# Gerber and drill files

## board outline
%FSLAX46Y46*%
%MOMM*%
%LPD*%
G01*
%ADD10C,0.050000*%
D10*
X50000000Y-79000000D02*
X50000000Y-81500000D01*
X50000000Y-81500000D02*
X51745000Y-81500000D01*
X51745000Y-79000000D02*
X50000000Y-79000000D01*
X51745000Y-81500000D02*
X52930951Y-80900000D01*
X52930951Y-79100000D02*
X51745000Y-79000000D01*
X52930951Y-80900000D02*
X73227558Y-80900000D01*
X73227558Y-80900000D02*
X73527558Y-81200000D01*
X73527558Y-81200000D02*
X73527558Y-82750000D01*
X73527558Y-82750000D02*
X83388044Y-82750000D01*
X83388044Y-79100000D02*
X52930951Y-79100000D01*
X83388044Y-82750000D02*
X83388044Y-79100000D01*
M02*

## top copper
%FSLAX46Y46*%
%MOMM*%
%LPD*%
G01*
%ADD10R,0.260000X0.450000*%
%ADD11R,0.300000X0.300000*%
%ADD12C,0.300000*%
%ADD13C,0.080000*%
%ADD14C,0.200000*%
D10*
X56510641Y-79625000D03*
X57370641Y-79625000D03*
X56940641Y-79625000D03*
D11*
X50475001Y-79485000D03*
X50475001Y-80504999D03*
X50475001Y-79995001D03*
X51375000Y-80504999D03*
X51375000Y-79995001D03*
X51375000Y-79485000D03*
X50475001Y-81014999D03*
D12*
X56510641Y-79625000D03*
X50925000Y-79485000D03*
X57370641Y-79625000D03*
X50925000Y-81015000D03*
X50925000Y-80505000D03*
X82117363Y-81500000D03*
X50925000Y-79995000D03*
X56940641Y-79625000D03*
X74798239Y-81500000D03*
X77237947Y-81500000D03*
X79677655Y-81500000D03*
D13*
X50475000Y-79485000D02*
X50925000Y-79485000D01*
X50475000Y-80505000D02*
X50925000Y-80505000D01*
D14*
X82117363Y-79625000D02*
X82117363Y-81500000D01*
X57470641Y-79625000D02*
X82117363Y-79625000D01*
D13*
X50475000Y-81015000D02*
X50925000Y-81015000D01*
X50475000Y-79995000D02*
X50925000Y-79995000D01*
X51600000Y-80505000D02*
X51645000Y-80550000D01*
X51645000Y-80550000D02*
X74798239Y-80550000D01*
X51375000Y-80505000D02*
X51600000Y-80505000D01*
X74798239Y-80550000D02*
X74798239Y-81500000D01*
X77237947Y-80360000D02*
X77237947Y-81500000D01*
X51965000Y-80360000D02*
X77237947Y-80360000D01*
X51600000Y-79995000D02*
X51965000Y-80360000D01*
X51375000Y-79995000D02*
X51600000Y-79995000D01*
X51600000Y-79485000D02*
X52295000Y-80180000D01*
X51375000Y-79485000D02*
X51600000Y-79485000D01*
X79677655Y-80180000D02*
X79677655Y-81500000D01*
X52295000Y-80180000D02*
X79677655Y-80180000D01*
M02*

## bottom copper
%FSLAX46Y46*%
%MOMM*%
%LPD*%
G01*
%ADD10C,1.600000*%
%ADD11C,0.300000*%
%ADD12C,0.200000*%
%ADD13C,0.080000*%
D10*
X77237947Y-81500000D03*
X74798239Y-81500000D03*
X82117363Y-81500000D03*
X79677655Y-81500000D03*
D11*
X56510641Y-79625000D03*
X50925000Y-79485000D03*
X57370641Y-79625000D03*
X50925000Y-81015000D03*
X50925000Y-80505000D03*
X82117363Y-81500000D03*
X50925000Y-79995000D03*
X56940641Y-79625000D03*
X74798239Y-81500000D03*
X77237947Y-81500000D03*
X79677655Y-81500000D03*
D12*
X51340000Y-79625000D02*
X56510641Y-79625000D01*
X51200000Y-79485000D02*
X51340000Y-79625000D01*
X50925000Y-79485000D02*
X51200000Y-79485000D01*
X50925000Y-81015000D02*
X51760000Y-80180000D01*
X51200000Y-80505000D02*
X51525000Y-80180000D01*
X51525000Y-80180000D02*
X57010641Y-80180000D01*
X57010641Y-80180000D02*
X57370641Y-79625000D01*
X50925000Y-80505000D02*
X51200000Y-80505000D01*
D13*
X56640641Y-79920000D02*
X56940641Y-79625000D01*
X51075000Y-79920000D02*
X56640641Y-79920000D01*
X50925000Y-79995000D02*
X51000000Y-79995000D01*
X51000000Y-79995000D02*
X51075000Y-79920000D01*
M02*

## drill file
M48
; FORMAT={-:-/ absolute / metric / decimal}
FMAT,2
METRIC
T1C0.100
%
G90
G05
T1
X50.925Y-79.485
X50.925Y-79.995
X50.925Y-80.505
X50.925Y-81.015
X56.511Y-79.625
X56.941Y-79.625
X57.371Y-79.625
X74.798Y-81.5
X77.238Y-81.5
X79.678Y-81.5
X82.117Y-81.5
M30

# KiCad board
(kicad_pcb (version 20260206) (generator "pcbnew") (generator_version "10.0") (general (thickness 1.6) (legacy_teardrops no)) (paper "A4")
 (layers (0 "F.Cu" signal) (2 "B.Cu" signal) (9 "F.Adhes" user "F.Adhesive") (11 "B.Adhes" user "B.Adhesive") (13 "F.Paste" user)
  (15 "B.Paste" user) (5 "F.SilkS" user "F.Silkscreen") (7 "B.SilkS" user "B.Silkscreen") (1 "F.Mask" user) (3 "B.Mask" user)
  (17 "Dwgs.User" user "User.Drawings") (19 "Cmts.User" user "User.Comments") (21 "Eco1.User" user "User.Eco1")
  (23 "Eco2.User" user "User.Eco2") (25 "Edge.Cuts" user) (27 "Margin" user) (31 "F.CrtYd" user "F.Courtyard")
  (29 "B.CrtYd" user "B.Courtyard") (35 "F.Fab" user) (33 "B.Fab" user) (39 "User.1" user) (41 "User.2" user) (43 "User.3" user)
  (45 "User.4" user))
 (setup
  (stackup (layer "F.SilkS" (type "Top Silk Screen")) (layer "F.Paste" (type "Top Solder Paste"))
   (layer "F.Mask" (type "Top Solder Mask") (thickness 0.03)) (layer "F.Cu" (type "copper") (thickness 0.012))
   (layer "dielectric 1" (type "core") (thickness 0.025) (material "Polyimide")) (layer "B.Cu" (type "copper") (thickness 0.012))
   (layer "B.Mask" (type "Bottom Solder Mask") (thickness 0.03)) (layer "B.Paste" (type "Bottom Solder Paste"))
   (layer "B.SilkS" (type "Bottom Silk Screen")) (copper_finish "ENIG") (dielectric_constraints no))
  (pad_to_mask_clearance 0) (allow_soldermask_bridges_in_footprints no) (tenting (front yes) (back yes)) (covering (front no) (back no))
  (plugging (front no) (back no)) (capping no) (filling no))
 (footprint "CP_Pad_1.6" (layer "F.Cu") (at 74.798239 81.5)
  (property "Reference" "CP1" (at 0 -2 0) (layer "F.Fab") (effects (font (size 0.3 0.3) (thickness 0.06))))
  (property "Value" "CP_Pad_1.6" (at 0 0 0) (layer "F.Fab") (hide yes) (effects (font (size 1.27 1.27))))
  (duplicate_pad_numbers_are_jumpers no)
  (pad "1" smd circle (at 0 0) (size 1.6 1.6) (layers "B.Cu" "B.Mask") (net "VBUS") (solder_mask_margin 0.1)))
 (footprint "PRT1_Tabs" (layer "F.Cu") (at 56.940641 79.625)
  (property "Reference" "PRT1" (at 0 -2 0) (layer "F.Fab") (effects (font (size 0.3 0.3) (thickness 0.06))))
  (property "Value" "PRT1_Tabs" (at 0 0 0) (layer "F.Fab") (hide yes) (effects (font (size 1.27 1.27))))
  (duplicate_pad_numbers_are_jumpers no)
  (pad "1" smd rect (at -0.43 0) (size 0.26 0.45) (layers "F.Cu" "F.Mask") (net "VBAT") (solder_mask_margin 0.05) (thermal_bridge_angle 45))
  (pad "2" smd rect (at 0.43 0) (size 0.26 0.45) (layers "F.Cu" "F.Mask") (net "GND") (solder_mask_margin 0.05) (thermal_bridge_angle 45))
  (pad "3" smd rect (at 0 0) (size 0.26 0.45) (layers "F.Cu" "F.Mask") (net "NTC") (solder_mask_margin 0.05) (thermal_bridge_angle 45)))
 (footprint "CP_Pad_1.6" (layer "F.Cu") (at 77.237947 81.5)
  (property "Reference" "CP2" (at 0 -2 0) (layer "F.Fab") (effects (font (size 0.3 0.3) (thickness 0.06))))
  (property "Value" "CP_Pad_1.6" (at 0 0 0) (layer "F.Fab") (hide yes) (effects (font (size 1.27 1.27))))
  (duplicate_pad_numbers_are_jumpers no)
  (pad "1" smd circle (at 0 0) (size 1.6 1.6) (layers "B.Cu" "B.Mask") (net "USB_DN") (solder_mask_margin 0.1)))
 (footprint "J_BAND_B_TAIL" (layer "F.Cu") (at 50.9 80.25)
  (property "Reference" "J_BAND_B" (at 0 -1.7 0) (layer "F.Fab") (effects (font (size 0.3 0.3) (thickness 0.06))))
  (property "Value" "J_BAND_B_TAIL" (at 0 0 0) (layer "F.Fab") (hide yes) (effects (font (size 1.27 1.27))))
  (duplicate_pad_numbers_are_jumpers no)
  (pad "1" smd rect (at -0.424999 -0.765) (size 0.3 0.3) (layers "F.Cu" "F.Mask") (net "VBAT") (solder_mask_margin 0.05)
   (thermal_bridge_angle 45))
  (pad "2" smd rect (at -0.424999 0.254999) (size 0.3 0.3) (layers "F.Cu" "F.Mask") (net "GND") (solder_mask_margin 0.05)
   (thermal_bridge_angle 45))
  (pad "3" smd rect (at -0.424999 -0.254999) (size 0.3 0.3) (layers "F.Cu" "F.Mask") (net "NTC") (solder_mask_margin 0.05)
   (thermal_bridge_angle 45))
  (pad "4" smd rect (at 0.475 0.254999) (size 0.3 0.3) (layers "F.Cu" "F.Mask") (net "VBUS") (solder_mask_margin 0.05)
   (thermal_bridge_angle 45))
  (pad "5" smd rect (at 0.475 -0.254999) (size 0.3 0.3) (layers "F.Cu" "F.Mask") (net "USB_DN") (solder_mask_margin 0.05)
   (thermal_bridge_angle 45))
  (pad "6" smd rect (at 0.475 -0.765) (size 0.3 0.3) (layers "F.Cu" "F.Mask") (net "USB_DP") (solder_mask_margin 0.05)
   (thermal_bridge_angle 45))
  (pad "7" smd rect (at -0.424999 0.764999) (size 0.3 0.3) (layers "F.Cu" "F.Mask") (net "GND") (solder_mask_margin 0.05)
   (thermal_bridge_angle 45)))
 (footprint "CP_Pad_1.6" (layer "F.Cu") (at 82.117363 81.5)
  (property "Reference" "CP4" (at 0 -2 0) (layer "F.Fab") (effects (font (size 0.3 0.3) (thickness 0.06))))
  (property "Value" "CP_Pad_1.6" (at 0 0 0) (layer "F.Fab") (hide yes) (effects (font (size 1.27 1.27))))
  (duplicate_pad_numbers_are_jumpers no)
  (pad "1" smd circle (at 0 0) (size 1.6 1.6) (layers "B.Cu" "B.Mask") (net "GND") (solder_mask_margin 0.1)))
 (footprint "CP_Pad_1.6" (layer "F.Cu") (at 79.677655 81.5)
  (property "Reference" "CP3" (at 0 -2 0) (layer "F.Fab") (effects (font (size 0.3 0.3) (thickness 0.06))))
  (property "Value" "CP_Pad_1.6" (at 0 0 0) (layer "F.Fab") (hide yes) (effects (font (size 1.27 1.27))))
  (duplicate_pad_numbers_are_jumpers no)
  (pad "1" smd circle (at 0 0) (size 1.6 1.6) (layers "B.Cu" "B.Mask") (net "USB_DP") (solder_mask_margin 0.1)))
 (gr_line (start 50 79) (end 50 81.5) (stroke (width 0.05) (type default)) (layer "Edge.Cuts"))
 (gr_line (start 50 81.5) (end 51.745 81.5) (stroke (width 0.05) (type default)) (layer "Edge.Cuts"))
 (gr_line (start 51.745 79) (end 50 79) (stroke (width 0.05) (type default)) (layer "Edge.Cuts"))
 (gr_line (start 51.745 81.5) (end 52.930951 80.9) (stroke (width 0.05) (type default)) (layer "Edge.Cuts"))
 (gr_line (start 52.930951 79.1) (end 51.745 79) (stroke (width 0.05) (type default)) (layer "Edge.Cuts"))
 (gr_line (start 52.930951 80.9) (end 73.227558 80.9) (stroke (width 0.05) (type default)) (layer "Edge.Cuts"))
 (gr_line (start 73.227558 80.9) (end 73.527558 81.2) (stroke (width 0.05) (type default)) (layer "Edge.Cuts"))
 (gr_line (start 73.527558 81.2) (end 73.527558 82.75) (stroke (width 0.05) (type default)) (layer "Edge.Cuts"))
 (gr_line (start 73.527558 82.75) (end 83.388044 82.75) (stroke (width 0.05) (type default)) (layer "Edge.Cuts"))
 (gr_line (start 83.388044 79.1) (end 52.930951 79.1) (stroke (width 0.05) (type default)) (layer "Edge.Cuts"))
 (gr_line (start 83.388044 82.75) (end 83.388044 79.1) (stroke (width 0.05) (type default)) (layer "Edge.Cuts"))
 (segment (start 50.475 79.485) (end 50.925 79.485) (width 0.08) (layer "F.Cu") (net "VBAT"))
 (via (at 56.510641 79.625) (size 0.3) (drill 0.1) (layers "F.Cu" "B.Cu") (tenting (front yes) (back yes)) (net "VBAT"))
 (via (at 50.925 79.485) (size 0.3) (drill 0.1) (layers "F.Cu" "B.Cu") (tenting (front yes) (back yes)) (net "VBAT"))
 (segment (start 51.2 79.485) (end 51.34 79.625) (width 0.2) (layer "B.Cu") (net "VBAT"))
 (segment (start 51.34 79.625) (end 56.510641 79.625) (width 0.2) (layer "B.Cu") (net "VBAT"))
 (segment (start 50.925 79.485) (end 51.2 79.485) (width 0.2) (layer "B.Cu") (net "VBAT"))
 (segment (start 82.117363 79.625) (end 82.117363 81.5) (width 0.2) (layer "F.Cu") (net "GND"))
 (segment (start 50.475 80.505) (end 50.925 80.505) (width 0.08) (layer "F.Cu") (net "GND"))
 (segment (start 57.470641 79.625) (end 82.117363 79.625) (width 0.2) (layer "F.Cu") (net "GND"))
 (segment (start 50.475 81.015) (end 50.925 81.015) (width 0.08) (layer "F.Cu") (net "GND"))
 (via (at 50.925 81.015) (size 0.3) (drill 0.1) (layers "F.Cu" "B.Cu") (tenting (front yes) (back yes)) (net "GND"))
 (via (at 57.370641 79.625) (size 0.3) (drill 0.1) (layers "F.Cu" "B.Cu") (tenting (front yes) (back yes)) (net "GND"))
 (via (at 82.117363 81.5) (size 0.3) (drill 0.1) (layers "F.Cu" "B.Cu") (tenting (front yes) (back yes)) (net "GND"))
 (via (at 50.925 80.505) (size 0.3) (drill 0.1) (layers "F.Cu" "B.Cu") (tenting (front yes) (back yes)) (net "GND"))
 (segment (start 50.925 81.015) (end 51.76 80.18) (width 0.2) (layer "B.Cu") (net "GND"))
 (segment (start 57.010641 80.18) (end 57.370641 79.625) (width 0.2) (layer "B.Cu") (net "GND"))
 (segment (start 51.525 80.18) (end 57.010641 80.18) (width 0.2) (layer "B.Cu") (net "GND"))
 (segment (start 51.2 80.505) (end 51.525 80.18) (width 0.2) (layer "B.Cu") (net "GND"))
 (segment (start 50.925 80.505) (end 51.2 80.505) (width 0.2) (layer "B.Cu") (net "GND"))
 (segment (start 50.475 79.995) (end 50.925 79.995) (width 0.08) (layer "F.Cu") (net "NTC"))
 (via (at 56.940641 79.625) (size 0.3) (drill 0.1) (layers "F.Cu" "B.Cu") (tenting (front yes) (back yes)) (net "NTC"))
 (via (at 50.925 79.995) (size 0.3) (drill 0.1) (layers "F.Cu" "B.Cu") (tenting (front yes) (back yes)) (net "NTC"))
 (segment (start 50.925 79.995) (end 51 79.995) (width 0.08) (layer "B.Cu") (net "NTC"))
 (segment (start 56.640641 79.92) (end 56.940641 79.625) (width 0.08) (layer "B.Cu") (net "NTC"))
 (segment (start 51.075 79.92) (end 56.640641 79.92) (width 0.08) (layer "B.Cu") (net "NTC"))
 (segment (start 51 79.995) (end 51.075 79.92) (width 0.08) (layer "B.Cu") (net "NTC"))
 (segment (start 51.645 80.55) (end 74.798239 80.55) (width 0.08) (layer "F.Cu") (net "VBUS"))
 (segment (start 51.6 80.505) (end 51.645 80.55) (width 0.08) (layer "F.Cu") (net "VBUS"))
 (segment (start 51.375 80.505) (end 51.6 80.505) (width 0.08) (layer "F.Cu") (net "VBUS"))
 (segment (start 74.798239 80.55) (end 74.798239 81.5) (width 0.08) (layer "F.Cu") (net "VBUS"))
 (via (at 74.798239 81.5) (size 0.3) (drill 0.1) (layers "F.Cu" "B.Cu") (tenting (front yes) (back yes)) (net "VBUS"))
 (segment (start 51.6 79.995) (end 51.965 80.36) (width 0.08) (layer "F.Cu") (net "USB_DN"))
 (segment (start 77.237947 80.36) (end 77.237947 81.5) (width 0.08) (layer "F.Cu") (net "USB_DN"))
 (segment (start 51.965 80.36) (end 77.237947 80.36) (width 0.08) (layer "F.Cu") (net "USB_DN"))
 (segment (start 51.375 79.995) (end 51.6 79.995) (width 0.08) (layer "F.Cu") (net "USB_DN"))
 (via (at 77.237947 81.5) (size 0.3) (drill 0.1) (layers "F.Cu" "B.Cu") (tenting (front yes) (back yes)) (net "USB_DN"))
 (segment (start 51.375 79.485) (end 51.6 79.485) (width 0.08) (layer "F.Cu") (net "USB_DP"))
 (segment (start 79.677655 80.18) (end 79.677655 81.5) (width 0.08) (layer "F.Cu") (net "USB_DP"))
 (segment (start 52.295 80.18) (end 79.677655 80.18) (width 0.08) (layer "F.Cu") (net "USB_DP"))
 (segment (start 51.6 79.485) (end 52.295 80.18) (width 0.08) (layer "F.Cu") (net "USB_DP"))
 (via (at 79.677655 81.5) (size 0.3) (drill 0.1) (layers "F.Cu" "B.Cu") (tenting (front yes) (back yes)) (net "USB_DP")))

